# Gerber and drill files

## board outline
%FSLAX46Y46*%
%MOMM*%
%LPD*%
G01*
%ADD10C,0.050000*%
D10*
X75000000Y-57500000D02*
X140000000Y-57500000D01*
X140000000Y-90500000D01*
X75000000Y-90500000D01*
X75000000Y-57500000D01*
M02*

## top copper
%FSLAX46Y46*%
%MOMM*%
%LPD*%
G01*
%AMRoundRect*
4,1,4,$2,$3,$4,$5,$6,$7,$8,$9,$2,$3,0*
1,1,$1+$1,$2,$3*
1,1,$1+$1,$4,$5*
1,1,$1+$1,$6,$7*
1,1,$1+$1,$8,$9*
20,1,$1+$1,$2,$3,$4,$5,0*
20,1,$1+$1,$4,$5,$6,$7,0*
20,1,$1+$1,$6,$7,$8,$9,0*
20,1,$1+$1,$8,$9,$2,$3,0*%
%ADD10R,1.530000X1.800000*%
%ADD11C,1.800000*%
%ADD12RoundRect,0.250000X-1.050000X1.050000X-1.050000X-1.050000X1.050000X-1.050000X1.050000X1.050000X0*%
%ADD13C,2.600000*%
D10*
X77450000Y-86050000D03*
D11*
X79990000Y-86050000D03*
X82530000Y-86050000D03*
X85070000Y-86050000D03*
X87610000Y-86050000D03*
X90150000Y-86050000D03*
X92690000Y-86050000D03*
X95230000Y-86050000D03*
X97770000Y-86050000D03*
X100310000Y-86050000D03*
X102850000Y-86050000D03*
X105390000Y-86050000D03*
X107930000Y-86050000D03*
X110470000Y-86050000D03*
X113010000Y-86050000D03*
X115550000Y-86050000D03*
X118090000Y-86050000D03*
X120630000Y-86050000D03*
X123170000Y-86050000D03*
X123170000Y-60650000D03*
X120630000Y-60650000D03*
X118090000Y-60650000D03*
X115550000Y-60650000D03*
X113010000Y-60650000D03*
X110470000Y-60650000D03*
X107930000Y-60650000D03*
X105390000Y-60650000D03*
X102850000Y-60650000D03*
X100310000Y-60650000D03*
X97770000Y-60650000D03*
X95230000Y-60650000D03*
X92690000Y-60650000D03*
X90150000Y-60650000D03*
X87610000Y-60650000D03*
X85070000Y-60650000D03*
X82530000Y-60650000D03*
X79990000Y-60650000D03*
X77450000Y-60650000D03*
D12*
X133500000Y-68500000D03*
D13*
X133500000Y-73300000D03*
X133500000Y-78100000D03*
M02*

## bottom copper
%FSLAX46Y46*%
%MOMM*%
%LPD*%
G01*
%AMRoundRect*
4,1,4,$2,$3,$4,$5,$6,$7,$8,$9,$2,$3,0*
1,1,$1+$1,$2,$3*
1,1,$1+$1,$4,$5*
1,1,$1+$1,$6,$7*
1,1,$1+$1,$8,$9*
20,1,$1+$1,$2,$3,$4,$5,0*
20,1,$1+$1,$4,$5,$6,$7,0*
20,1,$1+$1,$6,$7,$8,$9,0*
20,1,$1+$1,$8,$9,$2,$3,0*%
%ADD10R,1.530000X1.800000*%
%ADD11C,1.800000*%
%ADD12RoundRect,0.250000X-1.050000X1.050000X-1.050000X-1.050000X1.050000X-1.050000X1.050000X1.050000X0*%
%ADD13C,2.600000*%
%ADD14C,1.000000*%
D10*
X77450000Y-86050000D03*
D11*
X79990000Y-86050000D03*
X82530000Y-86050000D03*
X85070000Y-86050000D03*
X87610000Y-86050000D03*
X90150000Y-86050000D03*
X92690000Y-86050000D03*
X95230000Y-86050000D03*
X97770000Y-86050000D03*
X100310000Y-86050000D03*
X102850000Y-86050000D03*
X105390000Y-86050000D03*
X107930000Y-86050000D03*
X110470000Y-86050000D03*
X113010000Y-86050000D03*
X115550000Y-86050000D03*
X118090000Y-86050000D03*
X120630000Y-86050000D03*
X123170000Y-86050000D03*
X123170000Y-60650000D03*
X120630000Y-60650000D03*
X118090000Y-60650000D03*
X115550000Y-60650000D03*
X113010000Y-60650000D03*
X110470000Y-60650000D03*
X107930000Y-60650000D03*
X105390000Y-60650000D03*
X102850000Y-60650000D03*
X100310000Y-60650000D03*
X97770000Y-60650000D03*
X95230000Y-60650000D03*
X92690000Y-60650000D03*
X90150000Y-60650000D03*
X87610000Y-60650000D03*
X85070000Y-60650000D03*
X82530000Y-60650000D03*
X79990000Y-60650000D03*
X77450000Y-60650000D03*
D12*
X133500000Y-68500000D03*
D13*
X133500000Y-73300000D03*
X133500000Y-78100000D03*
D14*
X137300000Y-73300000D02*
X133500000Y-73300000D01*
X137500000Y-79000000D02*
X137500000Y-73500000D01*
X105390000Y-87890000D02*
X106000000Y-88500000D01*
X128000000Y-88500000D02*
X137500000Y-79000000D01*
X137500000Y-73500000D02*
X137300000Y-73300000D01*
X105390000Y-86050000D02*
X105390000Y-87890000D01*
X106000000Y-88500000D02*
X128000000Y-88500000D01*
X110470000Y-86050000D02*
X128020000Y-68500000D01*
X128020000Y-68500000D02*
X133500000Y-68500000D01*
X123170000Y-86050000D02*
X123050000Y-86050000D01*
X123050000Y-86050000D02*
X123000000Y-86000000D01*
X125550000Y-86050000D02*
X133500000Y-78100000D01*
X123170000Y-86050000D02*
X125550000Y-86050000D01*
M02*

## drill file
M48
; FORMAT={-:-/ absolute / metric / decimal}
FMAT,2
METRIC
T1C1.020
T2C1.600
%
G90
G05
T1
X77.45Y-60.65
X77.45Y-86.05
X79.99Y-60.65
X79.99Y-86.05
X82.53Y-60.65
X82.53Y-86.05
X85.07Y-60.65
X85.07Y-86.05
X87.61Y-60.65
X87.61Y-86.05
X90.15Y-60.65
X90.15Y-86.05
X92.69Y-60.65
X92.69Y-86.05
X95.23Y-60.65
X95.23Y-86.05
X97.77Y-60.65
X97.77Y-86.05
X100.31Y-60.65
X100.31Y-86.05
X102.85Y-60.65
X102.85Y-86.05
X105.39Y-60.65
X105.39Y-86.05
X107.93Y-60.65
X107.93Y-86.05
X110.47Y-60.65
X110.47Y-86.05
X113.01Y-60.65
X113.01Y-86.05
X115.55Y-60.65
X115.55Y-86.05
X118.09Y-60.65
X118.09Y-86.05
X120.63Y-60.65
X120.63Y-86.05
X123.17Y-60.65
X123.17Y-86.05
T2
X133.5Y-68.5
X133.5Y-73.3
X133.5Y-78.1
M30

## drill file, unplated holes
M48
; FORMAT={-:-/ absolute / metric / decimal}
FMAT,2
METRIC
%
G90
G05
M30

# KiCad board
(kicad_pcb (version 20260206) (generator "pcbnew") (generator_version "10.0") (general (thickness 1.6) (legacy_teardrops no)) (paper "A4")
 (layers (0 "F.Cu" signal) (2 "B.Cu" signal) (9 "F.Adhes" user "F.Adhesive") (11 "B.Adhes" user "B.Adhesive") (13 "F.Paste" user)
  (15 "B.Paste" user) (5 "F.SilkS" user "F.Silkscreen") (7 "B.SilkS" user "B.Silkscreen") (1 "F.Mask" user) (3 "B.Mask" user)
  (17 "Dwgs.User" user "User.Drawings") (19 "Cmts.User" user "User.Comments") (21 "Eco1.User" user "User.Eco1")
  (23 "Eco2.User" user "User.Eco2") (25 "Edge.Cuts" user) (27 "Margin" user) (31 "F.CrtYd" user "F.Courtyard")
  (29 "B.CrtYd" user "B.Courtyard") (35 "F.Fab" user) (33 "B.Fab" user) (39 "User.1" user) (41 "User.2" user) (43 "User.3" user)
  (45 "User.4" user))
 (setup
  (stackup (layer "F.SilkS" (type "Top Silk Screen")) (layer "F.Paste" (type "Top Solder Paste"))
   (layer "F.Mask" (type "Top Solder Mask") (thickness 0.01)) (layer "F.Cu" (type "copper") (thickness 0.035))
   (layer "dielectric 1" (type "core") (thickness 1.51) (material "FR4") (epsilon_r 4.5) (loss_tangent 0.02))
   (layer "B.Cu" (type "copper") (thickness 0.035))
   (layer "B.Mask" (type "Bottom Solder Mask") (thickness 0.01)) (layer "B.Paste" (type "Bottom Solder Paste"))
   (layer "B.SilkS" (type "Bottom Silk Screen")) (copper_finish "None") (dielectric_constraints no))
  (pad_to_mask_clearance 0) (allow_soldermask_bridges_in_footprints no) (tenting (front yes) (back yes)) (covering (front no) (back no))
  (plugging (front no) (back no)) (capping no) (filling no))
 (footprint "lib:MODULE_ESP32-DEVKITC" (layer "F.Cu") (at 100.3 73.35 90)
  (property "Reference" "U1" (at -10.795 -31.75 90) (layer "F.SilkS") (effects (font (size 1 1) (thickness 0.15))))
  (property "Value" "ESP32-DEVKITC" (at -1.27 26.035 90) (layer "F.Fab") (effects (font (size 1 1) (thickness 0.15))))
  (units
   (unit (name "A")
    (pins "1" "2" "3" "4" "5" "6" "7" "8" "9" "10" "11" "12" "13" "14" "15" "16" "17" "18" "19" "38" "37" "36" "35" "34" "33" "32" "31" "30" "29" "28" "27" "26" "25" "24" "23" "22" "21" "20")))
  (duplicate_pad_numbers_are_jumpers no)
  (pad "1" thru_hole rect (at -12.7 -22.85 90) (size 1.8 1.53) (drill 1.02) (layers "*.Cu" "*.Mask") (remove_unused_layers no)
   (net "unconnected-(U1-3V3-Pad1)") (solder_mask_margin 0.102))
  (pad "2" thru_hole circle (at -12.7 -20.31 90) (size 1.8 1.8) (drill 1.02) (layers "*.Cu" "*.Mask") (remove_unused_layers no)
   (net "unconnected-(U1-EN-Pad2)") (solder_mask_margin 0.102))
  (pad "3" thru_hole circle (at -12.7 -17.77 90) (size 1.8 1.8) (drill 1.02) (layers "*.Cu" "*.Mask") (remove_unused_layers no)
   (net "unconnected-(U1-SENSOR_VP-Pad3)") (solder_mask_margin 0.102))
  (pad "4" thru_hole circle (at -12.7 -15.23 90) (size 1.8 1.8) (drill 1.02) (layers "*.Cu" "*.Mask") (remove_unused_layers no)
   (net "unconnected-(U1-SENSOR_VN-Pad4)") (solder_mask_margin 0.102))
  (pad "5" thru_hole circle (at -12.7 -12.69 90) (size 1.8 1.8) (drill 1.02) (layers "*.Cu" "*.Mask") (remove_unused_layers no)
   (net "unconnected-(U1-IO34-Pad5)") (solder_mask_margin 0.102))
  (pad "6" thru_hole circle (at -12.7 -10.15 90) (size 1.8 1.8) (drill 1.02) (layers "*.Cu" "*.Mask") (remove_unused_layers no)
   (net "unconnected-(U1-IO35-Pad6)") (solder_mask_margin 0.102))
  (pad "7" thru_hole circle (at -12.7 -7.61 90) (size 1.8 1.8) (drill 1.02) (layers "*.Cu" "*.Mask") (remove_unused_layers no)
   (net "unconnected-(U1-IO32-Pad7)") (solder_mask_margin 0.102))
  (pad "8" thru_hole circle (at -12.7 -5.07 90) (size 1.8 1.8) (drill 1.02) (layers "*.Cu" "*.Mask") (remove_unused_layers no)
   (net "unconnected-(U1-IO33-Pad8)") (solder_mask_margin 0.102))
  (pad "9" thru_hole circle (at -12.7 -2.53 90) (size 1.8 1.8) (drill 1.02) (layers "*.Cu" "*.Mask") (remove_unused_layers no)
   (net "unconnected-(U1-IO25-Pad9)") (solder_mask_margin 0.102))
  (pad "10" thru_hole circle (at -12.7 0.01 90) (size 1.8 1.8) (drill 1.02) (layers "*.Cu" "*.Mask") (remove_unused_layers no)
   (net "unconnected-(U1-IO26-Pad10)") (solder_mask_margin 0.102))
  (pad "11" thru_hole circle (at -12.7 2.55 90) (size 1.8 1.8) (drill 1.02) (layers "*.Cu" "*.Mask") (remove_unused_layers no)
   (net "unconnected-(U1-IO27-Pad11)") (solder_mask_margin 0.102))
  (pad "12" thru_hole circle (at -12.7 5.09 90) (size 1.8 1.8) (drill 1.02) (layers "*.Cu" "*.Mask") (remove_unused_layers no)
   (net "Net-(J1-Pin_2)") (solder_mask_margin 0.102))
  (pad "13" thru_hole circle (at -12.7 7.63 90) (size 1.8 1.8) (drill 1.02) (layers "*.Cu" "*.Mask") (remove_unused_layers no)
   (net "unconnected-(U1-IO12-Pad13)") (solder_mask_margin 0.102))
  (pad "14" thru_hole circle (at -12.7 10.17 90) (size 1.8 1.8) (drill 1.02) (layers "*.Cu" "*.Mask") (remove_unused_layers no)
   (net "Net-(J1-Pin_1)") (solder_mask_margin 0.102))
  (pad "15" thru_hole circle (at -12.7 12.71 90) (size 1.8 1.8) (drill 1.02) (layers "*.Cu" "*.Mask") (remove_unused_layers no)
   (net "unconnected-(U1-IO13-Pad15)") (solder_mask_margin 0.102))
  (pad "16" thru_hole circle (at -12.7 15.25 90) (size 1.8 1.8) (drill 1.02) (layers "*.Cu" "*.Mask") (remove_unused_layers no)
   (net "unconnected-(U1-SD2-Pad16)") (solder_mask_margin 0.102))
  (pad "17" thru_hole circle (at -12.7 17.79 90) (size 1.8 1.8) (drill 1.02) (layers "*.Cu" "*.Mask") (remove_unused_layers no)
   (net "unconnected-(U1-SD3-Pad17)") (solder_mask_margin 0.102))
  (pad "18" thru_hole circle (at -12.7 20.33 90) (size 1.8 1.8) (drill 1.02) (layers "*.Cu" "*.Mask") (remove_unused_layers no)
   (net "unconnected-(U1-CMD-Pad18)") (solder_mask_margin 0.102))
  (pad "19" thru_hole circle (at -12.7 22.87 90) (size 1.8 1.8) (drill 1.02) (layers "*.Cu" "*.Mask") (remove_unused_layers no)
   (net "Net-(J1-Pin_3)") (solder_mask_margin 0.102))
  (pad "20" thru_hole circle (at 12.7 22.87 90) (size 1.8 1.8) (drill 1.02) (layers "*.Cu" "*.Mask") (remove_unused_layers no)
   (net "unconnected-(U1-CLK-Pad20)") (solder_mask_margin 0.102))
  (pad "21" thru_hole circle (at 12.7 20.33 90) (size 1.8 1.8) (drill 1.02) (layers "*.Cu" "*.Mask") (remove_unused_layers no)
   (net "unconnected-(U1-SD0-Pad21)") (solder_mask_margin 0.102))
  (pad "22" thru_hole circle (at 12.7 17.79 90) (size 1.8 1.8) (drill 1.02) (layers "*.Cu" "*.Mask") (remove_unused_layers no)
   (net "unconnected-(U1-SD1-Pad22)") (solder_mask_margin 0.102))
  (pad "23" thru_hole circle (at 12.7 15.25 90) (size 1.8 1.8) (drill 1.02) (layers "*.Cu" "*.Mask") (remove_unused_layers no)
   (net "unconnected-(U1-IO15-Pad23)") (solder_mask_margin 0.102))
  (pad "24" thru_hole circle (at 12.7 12.71 90) (size 1.8 1.8) (drill 1.02) (layers "*.Cu" "*.Mask") (remove_unused_layers no)
   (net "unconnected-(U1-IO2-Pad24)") (solder_mask_margin 0.102))
  (pad "25" thru_hole circle (at 12.7 10.17 90) (size 1.8 1.8) (drill 1.02) (layers "*.Cu" "*.Mask") (remove_unused_layers no)
   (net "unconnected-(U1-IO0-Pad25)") (solder_mask_margin 0.102))
  (pad "26" thru_hole circle (at 12.7 7.63 90) (size 1.8 1.8) (drill 1.02) (layers "*.Cu" "*.Mask") (remove_unused_layers no)
   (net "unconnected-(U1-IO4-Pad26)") (solder_mask_margin 0.102))
  (pad "27" thru_hole circle (at 12.7 5.09 90) (size 1.8 1.8) (drill 1.02) (layers "*.Cu" "*.Mask") (remove_unused_layers no)
   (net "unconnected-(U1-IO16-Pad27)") (solder_mask_margin 0.102))
  (pad "28" thru_hole circle (at 12.7 2.55 90) (size 1.8 1.8) (drill 1.02) (layers "*.Cu" "*.Mask") (remove_unused_layers no)
   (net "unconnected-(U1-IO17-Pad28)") (solder_mask_margin 0.102))
  (pad "29" thru_hole circle (at 12.7 0.01 90) (size 1.8 1.8) (drill 1.02) (layers "*.Cu" "*.Mask") (remove_unused_layers no)
   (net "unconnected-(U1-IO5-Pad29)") (solder_mask_margin 0.102))
  (pad "30" thru_hole circle (at 12.7 -2.53 90) (size 1.8 1.8) (drill 1.02) (layers "*.Cu" "*.Mask") (remove_unused_layers no)
   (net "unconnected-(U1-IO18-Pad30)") (solder_mask_margin 0.102))
  (pad "31" thru_hole circle (at 12.7 -5.07 90) (size 1.8 1.8) (drill 1.02) (layers "*.Cu" "*.Mask") (remove_unused_layers no)
   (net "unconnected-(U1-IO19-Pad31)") (solder_mask_margin 0.102))
  (pad "32" thru_hole circle (at 12.7 -7.61 90) (size 1.8 1.8) (drill 1.02) (layers "*.Cu" "*.Mask") (remove_unused_layers no)
   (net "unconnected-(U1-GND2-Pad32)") (solder_mask_margin 0.102))
  (pad "33" thru_hole circle (at 12.7 -10.15 90) (size 1.8 1.8) (drill 1.02) (layers "*.Cu" "*.Mask") (remove_unused_layers no)
   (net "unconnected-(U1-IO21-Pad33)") (solder_mask_margin 0.102))
  (pad "34" thru_hole circle (at 12.7 -12.69 90) (size 1.8 1.8) (drill 1.02) (layers "*.Cu" "*.Mask") (remove_unused_layers no)
   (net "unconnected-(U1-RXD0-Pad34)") (solder_mask_margin 0.102))
  (pad "35" thru_hole circle (at 12.7 -15.23 90) (size 1.8 1.8) (drill 1.02) (layers "*.Cu" "*.Mask") (remove_unused_layers no)
   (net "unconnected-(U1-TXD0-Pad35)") (solder_mask_margin 0.102))
  (pad "36" thru_hole circle (at 12.7 -17.77 90) (size 1.8 1.8) (drill 1.02) (layers "*.Cu" "*.Mask") (remove_unused_layers no)
   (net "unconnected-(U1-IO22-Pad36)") (solder_mask_margin 0.102))
  (pad "37" thru_hole circle (at 12.7 -20.31 90) (size 1.8 1.8) (drill 1.02) (layers "*.Cu" "*.Mask") (remove_unused_layers no)
   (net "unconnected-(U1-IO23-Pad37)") (solder_mask_margin 0.102))
  (pad "38" thru_hole circle (at 12.7 -22.85 90) (size 1.8 1.8) (drill 1.02) (layers "*.Cu" "*.Mask") (remove_unused_layers no)
   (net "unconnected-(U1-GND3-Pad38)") (solder_mask_margin 0.102)))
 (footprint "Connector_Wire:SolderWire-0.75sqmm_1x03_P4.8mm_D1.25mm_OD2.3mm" (layer "F.Cu") (at 133.5 68.5 -90)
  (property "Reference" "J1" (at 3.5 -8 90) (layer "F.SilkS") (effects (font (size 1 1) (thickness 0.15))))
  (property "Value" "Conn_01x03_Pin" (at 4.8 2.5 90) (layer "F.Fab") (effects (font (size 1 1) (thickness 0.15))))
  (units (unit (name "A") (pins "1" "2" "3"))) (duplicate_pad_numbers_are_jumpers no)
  (pad "1" thru_hole roundrect (at 0 0 270) (size 2.6 2.6) (drill 1.6) (layers "*.Cu" "*.Mask") (remove_unused_layers no)
   (roundrect_rratio 0.096154) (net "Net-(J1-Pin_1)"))
  (pad "2" thru_hole circle (at 4.8 0 270) (size 2.6 2.6) (drill 1.6) (layers "*.Cu" "*.Mask") (remove_unused_layers no)
   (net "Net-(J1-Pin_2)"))
  (pad "3" thru_hole circle (at 9.6 0 270) (size 2.6 2.6) (drill 1.6) (layers "*.Cu" "*.Mask") (remove_unused_layers no)
   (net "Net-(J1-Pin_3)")))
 (gr_rect (start 75 57.5) (end 140 90.5) (stroke (width 0.05) (type default)) (fill no) (layer "Edge.Cuts"))
 (segment (start 137.3 73.3) (end 133.5 73.3) (width 1) (layer "B.Cu") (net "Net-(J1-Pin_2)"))
 (segment (start 137.5 79) (end 137.5 73.5) (width 1) (layer "B.Cu") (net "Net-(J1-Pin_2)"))
 (segment (start 105.39 87.89) (end 106 88.5) (width 1) (layer "B.Cu") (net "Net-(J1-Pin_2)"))
 (segment (start 128 88.5) (end 137.5 79) (width 1) (layer "B.Cu") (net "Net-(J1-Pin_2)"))
 (segment (start 137.5 73.5) (end 137.3 73.3) (width 1) (layer "B.Cu") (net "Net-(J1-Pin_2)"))
 (segment (start 105.39 86.05) (end 105.39 87.89) (width 1) (layer "B.Cu") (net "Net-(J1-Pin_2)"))
 (segment (start 106 88.5) (end 128 88.5) (width 1) (layer "B.Cu") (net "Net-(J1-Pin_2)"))
 (segment (start 110.47 86.05) (end 128.02 68.5) (width 1) (layer "B.Cu") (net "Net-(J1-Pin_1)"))
 (segment (start 128.02 68.5) (end 133.5 68.5) (width 1) (layer "B.Cu") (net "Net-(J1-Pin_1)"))
 (segment (start 123.17 86.05) (end 123.05 86.05) (width 1) (layer "B.Cu") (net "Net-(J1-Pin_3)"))
 (segment (start 123.05 86.05) (end 123 86) (width 1) (layer "B.Cu") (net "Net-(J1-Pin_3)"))
 (segment (start 125.55 86.05) (end 133.5 78.1) (width 1) (layer "B.Cu") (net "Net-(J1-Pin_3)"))
 (segment (start 123.17 86.05) (end 125.55 86.05) (width 1) (layer "B.Cu") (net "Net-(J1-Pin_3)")))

